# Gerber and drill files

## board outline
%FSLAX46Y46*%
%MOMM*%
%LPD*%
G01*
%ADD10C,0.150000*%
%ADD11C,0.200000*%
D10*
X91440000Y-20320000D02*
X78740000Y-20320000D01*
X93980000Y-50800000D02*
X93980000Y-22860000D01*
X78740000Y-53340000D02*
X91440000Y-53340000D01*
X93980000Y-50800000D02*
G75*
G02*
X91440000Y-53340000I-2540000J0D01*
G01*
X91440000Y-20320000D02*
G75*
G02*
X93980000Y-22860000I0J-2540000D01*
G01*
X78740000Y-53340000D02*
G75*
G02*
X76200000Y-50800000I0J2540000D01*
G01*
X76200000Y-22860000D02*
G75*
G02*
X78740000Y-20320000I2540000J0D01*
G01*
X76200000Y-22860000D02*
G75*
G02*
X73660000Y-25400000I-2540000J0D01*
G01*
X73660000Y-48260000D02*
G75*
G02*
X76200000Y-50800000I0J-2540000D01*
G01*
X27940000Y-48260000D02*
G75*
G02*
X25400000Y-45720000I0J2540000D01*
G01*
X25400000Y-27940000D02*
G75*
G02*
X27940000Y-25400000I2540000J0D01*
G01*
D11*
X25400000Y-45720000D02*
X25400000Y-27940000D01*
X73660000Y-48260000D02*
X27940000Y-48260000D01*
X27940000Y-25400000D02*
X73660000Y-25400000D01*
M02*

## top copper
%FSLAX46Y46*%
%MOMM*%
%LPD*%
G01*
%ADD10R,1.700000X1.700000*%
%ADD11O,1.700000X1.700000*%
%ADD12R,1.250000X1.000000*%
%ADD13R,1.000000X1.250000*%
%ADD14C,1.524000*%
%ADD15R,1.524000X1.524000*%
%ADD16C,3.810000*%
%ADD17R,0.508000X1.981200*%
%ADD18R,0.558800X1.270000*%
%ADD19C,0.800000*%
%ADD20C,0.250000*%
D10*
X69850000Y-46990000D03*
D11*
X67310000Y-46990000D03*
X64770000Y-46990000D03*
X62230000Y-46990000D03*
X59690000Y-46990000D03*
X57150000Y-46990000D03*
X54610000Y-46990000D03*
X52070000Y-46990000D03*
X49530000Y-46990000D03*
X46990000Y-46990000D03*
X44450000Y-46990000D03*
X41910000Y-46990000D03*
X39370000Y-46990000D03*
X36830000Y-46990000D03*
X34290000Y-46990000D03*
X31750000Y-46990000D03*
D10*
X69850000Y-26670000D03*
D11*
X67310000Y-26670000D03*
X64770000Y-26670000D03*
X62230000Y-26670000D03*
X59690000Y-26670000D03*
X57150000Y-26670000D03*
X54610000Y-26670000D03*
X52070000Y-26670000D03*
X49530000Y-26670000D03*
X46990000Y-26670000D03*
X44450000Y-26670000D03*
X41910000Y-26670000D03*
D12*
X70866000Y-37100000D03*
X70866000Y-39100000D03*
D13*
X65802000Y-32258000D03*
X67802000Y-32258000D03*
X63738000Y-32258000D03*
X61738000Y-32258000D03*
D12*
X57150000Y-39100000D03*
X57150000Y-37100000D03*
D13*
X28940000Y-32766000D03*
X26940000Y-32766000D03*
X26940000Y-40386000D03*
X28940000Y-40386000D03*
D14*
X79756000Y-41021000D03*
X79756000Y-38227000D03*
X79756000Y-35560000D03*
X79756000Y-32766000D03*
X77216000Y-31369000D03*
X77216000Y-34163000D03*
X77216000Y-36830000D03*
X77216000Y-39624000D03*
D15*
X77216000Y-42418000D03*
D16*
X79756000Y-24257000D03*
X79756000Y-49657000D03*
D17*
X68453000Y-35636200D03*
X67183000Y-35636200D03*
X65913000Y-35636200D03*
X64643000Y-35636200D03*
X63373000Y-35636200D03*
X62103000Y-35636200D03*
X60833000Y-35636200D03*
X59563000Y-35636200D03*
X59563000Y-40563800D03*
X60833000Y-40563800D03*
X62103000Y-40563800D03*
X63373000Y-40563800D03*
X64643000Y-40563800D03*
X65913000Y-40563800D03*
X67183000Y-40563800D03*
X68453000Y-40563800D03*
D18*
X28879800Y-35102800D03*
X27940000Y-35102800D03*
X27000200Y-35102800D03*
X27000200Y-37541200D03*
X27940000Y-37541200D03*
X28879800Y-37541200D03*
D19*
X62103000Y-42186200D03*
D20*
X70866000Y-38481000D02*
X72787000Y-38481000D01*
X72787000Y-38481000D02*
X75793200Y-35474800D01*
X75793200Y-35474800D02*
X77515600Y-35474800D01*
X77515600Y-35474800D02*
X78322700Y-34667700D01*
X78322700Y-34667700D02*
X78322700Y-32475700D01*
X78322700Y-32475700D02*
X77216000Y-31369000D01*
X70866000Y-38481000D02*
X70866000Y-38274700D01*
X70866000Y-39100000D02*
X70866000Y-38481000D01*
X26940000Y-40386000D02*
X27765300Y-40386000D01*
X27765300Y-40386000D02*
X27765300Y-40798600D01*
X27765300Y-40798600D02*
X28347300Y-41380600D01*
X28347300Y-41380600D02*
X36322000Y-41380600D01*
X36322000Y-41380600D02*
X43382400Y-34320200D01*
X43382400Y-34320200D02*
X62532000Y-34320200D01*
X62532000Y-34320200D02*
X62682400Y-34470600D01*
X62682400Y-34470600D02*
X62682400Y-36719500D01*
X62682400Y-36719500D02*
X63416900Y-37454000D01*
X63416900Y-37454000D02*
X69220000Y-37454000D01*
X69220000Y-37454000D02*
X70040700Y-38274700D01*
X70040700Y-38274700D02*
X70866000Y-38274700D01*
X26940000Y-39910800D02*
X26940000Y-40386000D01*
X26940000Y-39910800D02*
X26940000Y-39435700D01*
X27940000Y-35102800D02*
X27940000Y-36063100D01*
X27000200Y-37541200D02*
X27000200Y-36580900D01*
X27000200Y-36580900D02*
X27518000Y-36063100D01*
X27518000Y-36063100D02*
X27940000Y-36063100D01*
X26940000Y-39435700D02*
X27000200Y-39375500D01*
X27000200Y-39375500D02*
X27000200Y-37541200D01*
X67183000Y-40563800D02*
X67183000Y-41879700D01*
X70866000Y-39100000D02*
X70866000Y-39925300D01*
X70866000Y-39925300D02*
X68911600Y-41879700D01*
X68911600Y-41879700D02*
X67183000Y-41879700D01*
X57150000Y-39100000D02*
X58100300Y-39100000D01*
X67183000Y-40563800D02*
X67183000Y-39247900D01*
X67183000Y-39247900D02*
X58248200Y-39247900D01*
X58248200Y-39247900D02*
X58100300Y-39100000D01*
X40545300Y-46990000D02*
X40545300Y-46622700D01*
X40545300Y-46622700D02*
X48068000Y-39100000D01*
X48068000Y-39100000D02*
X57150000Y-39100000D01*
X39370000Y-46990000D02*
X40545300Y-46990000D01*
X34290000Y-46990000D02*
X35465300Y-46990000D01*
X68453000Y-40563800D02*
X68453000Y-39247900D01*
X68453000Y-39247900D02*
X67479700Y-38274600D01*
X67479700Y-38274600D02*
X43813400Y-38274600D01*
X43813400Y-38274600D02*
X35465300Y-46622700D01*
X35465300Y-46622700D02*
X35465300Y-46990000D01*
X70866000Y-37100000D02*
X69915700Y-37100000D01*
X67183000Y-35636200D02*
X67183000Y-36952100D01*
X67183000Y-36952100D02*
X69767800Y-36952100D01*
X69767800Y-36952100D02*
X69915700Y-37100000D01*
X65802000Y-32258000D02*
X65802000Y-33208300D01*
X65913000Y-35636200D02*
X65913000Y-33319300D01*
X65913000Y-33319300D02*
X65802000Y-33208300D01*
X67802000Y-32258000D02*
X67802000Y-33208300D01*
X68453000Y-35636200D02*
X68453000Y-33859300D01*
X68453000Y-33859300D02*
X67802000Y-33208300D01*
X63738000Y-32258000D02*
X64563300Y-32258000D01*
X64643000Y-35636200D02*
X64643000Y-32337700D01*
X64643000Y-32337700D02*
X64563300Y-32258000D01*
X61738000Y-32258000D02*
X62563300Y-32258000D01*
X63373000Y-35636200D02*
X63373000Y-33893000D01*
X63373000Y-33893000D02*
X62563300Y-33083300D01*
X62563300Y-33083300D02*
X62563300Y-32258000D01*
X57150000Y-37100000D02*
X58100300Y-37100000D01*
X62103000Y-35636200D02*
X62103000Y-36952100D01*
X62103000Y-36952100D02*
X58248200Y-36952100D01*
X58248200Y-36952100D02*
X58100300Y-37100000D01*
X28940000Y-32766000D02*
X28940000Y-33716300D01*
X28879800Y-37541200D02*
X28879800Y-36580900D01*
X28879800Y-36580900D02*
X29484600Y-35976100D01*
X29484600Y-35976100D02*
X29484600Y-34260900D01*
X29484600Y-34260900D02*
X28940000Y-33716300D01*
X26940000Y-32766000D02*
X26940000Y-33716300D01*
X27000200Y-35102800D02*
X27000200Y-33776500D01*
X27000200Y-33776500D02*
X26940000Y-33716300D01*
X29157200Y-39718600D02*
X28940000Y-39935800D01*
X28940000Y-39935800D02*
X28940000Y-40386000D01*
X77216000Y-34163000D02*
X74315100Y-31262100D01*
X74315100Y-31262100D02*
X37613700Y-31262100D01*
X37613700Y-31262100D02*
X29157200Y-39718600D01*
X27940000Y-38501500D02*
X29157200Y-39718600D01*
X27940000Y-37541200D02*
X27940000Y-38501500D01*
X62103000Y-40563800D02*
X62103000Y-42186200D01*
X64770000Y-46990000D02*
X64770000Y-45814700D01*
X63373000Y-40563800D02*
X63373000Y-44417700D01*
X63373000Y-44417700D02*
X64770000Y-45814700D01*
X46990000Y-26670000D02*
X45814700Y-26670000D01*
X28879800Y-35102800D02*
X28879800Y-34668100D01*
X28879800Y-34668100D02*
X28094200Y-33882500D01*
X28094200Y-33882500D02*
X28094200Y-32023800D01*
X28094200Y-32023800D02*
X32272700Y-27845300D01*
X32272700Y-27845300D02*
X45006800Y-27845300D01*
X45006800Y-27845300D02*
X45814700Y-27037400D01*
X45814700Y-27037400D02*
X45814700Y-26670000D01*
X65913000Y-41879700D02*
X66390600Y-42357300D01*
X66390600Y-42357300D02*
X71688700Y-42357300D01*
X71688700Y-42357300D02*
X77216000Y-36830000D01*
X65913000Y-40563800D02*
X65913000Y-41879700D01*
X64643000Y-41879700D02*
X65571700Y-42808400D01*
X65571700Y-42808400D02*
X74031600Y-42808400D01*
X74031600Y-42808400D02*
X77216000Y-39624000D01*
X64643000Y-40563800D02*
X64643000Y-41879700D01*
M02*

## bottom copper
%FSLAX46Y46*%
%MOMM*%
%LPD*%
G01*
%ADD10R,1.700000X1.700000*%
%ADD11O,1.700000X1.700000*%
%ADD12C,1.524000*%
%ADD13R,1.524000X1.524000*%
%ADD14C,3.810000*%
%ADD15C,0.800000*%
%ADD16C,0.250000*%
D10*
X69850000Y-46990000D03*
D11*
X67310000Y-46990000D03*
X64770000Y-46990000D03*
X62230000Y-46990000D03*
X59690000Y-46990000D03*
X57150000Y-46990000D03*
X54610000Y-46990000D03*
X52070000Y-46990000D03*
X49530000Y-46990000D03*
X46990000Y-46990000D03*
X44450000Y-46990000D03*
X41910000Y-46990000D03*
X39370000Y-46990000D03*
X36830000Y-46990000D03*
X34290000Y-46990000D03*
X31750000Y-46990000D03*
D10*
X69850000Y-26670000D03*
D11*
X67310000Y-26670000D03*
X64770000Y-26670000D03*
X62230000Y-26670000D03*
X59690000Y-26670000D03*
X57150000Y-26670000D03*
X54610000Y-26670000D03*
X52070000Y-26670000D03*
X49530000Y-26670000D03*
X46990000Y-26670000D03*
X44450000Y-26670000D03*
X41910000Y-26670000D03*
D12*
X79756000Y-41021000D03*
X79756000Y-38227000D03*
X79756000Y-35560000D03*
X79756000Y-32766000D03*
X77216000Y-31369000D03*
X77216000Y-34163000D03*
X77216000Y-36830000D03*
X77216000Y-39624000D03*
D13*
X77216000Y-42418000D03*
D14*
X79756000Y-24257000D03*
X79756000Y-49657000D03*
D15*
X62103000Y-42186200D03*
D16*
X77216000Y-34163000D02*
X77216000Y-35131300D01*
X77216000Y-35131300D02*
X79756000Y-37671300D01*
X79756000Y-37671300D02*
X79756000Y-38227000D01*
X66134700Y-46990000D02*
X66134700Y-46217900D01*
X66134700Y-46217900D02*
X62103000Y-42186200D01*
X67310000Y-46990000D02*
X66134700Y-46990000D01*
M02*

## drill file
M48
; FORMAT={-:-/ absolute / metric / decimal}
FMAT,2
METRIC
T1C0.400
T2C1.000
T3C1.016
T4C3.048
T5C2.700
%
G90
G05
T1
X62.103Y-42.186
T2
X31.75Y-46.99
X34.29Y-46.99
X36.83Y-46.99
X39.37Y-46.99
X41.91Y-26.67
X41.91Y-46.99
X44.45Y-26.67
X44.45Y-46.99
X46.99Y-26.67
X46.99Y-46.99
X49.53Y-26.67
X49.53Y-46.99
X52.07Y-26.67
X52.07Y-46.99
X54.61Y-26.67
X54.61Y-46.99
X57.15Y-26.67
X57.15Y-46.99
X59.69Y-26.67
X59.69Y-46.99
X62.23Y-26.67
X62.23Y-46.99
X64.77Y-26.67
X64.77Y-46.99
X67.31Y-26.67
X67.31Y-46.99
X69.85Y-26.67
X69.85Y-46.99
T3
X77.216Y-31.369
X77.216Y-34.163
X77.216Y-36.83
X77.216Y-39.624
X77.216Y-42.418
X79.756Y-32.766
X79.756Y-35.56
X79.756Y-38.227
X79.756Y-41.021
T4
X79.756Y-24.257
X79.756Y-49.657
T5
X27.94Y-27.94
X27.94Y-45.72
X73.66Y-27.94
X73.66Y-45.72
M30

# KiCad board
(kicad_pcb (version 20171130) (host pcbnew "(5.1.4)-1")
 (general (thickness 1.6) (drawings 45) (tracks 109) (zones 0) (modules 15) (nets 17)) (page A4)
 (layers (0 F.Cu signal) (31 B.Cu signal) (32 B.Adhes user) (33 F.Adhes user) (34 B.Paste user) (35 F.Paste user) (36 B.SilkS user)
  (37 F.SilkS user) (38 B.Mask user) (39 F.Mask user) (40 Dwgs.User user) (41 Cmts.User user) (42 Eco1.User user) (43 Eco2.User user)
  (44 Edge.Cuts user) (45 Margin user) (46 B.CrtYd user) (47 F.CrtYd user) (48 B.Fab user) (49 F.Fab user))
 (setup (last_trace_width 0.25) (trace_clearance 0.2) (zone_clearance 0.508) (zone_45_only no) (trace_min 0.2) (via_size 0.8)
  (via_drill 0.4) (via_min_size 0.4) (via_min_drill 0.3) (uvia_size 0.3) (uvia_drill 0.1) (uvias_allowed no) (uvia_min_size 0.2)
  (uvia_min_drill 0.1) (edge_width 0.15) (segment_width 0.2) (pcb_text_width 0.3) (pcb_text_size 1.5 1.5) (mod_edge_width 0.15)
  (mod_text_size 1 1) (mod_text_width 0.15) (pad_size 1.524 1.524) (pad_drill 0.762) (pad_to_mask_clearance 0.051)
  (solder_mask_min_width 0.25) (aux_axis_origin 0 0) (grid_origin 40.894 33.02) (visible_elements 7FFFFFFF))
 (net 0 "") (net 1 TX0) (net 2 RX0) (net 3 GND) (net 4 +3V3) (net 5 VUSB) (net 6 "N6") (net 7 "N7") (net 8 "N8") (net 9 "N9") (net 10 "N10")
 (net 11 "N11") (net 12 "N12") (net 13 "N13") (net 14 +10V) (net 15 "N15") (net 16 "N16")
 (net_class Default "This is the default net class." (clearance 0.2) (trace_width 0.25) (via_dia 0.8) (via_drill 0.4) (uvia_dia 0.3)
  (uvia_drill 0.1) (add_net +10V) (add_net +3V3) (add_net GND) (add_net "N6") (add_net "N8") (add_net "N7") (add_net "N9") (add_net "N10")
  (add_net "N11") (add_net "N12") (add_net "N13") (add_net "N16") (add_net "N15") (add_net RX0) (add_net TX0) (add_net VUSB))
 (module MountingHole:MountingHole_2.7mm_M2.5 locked (layer F.Cu) (at 73.66 27.94)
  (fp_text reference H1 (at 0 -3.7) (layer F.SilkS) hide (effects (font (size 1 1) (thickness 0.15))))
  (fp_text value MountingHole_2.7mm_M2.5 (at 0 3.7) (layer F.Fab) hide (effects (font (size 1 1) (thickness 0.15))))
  (pad 1 np_thru_hole circle (at 0 0) (size 2.7 2.7) (drill 2.7) (layers *.Cu *.Mask)))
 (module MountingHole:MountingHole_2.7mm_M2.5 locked (layer F.Cu) (at 73.66 45.72)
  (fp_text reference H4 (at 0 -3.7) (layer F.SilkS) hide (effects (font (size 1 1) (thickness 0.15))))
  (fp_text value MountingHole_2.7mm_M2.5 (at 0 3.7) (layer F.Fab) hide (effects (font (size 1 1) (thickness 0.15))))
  (pad 1 np_thru_hole circle (at 0 0) (size 2.7 2.7) (drill 2.7) (layers *.Cu *.Mask)))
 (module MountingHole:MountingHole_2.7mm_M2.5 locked (layer F.Cu) (at 27.94 45.72)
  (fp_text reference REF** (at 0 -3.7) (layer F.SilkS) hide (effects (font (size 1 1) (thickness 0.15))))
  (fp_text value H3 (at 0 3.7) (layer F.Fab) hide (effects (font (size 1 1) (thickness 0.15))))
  (pad 1 np_thru_hole circle (at 0 0) (size 2.7 2.7) (drill 2.7) (layers *.Cu *.Mask)))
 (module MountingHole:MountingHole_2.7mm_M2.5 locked (layer F.Cu) (at 27.94 27.94)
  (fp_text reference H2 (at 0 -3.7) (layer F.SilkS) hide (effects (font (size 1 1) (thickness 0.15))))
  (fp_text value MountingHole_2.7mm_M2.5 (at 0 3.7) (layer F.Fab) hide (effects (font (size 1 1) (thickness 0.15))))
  (pad 1 np_thru_hole circle (at 0 0) (size 2.7 2.7) (drill 2.7) (layers *.Cu *.Mask)))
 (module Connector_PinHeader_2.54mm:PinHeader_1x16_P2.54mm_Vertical (layer B.Cu) (at 69.85 46.99 90)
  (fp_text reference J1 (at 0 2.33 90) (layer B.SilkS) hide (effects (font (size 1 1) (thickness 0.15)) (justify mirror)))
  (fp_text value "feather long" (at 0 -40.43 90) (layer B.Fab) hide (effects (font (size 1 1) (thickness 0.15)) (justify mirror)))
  (pad 1 thru_hole rect (at 0 0 90) (size 1.7 1.7) (drill 1) (layers *.Cu *.Mask))
  (pad 2 thru_hole oval (at 0 -2.54 90) (size 1.7 1.7) (drill 1) (layers *.Cu *.Mask) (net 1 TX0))
  (pad 3 thru_hole oval (at 0 -5.08 90) (size 1.7 1.7) (drill 1) (layers *.Cu *.Mask) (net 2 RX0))
  (pad 4 thru_hole oval (at 0 -7.62 90) (size 1.7 1.7) (drill 1) (layers *.Cu *.Mask))
  (pad 5 thru_hole oval (at 0 -10.16 90) (size 1.7 1.7) (drill 1) (layers *.Cu *.Mask))
  (pad 6 thru_hole oval (at 0 -12.7 90) (size 1.7 1.7) (drill 1) (layers *.Cu *.Mask))
  (pad 7 thru_hole oval (at 0 -15.24 90) (size 1.7 1.7) (drill 1) (layers *.Cu *.Mask))
  (pad 8 thru_hole oval (at 0 -17.78 90) (size 1.7 1.7) (drill 1) (layers *.Cu *.Mask))
  (pad 9 thru_hole oval (at 0 -20.32 90) (size 1.7 1.7) (drill 1) (layers *.Cu *.Mask))
  (pad 10 thru_hole oval (at 0 -22.86 90) (size 1.7 1.7) (drill 1) (layers *.Cu *.Mask))
  (pad 11 thru_hole oval (at 0 -25.4 90) (size 1.7 1.7) (drill 1) (layers *.Cu *.Mask))
  (pad 12 thru_hole oval (at 0 -27.94 90) (size 1.7 1.7) (drill 1) (layers *.Cu *.Mask))
  (pad 13 thru_hole oval (at 0 -30.48 90) (size 1.7 1.7) (drill 1) (layers *.Cu *.Mask) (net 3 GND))
  (pad 14 thru_hole oval (at 0 -33.02 90) (size 1.7 1.7) (drill 1) (layers *.Cu *.Mask))
  (pad 15 thru_hole oval (at 0 -35.56 90) (size 1.7 1.7) (drill 1) (layers *.Cu *.Mask) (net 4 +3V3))
  (pad 16 thru_hole oval (at 0 -38.1 90) (size 1.7 1.7) (drill 1) (layers *.Cu *.Mask)))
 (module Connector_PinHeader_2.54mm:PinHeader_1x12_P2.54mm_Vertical (layer B.Cu) (at 69.85 26.67 90)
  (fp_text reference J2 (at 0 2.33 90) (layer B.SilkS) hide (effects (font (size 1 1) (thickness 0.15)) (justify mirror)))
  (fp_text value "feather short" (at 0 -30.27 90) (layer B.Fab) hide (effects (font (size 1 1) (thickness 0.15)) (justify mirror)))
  (pad 1 thru_hole rect (at 0 0 90) (size 1.7 1.7) (drill 1) (layers *.Cu *.Mask))
  (pad 2 thru_hole oval (at 0 -2.54 90) (size 1.7 1.7) (drill 1) (layers *.Cu *.Mask))
  (pad 3 thru_hole oval (at 0 -5.08 90) (size 1.7 1.7) (drill 1) (layers *.Cu *.Mask))
  (pad 4 thru_hole oval (at 0 -7.62 90) (size 1.7 1.7) (drill 1) (layers *.Cu *.Mask))
  (pad 5 thru_hole oval (at 0 -10.16 90) (size 1.7 1.7) (drill 1) (layers *.Cu *.Mask))
  (pad 6 thru_hole oval (at 0 -12.7 90) (size 1.7 1.7) (drill 1) (layers *.Cu *.Mask))
  (pad 7 thru_hole oval (at 0 -15.24 90) (size 1.7 1.7) (drill 1) (layers *.Cu *.Mask))
  (pad 8 thru_hole oval (at 0 -17.78 90) (size 1.7 1.7) (drill 1) (layers *.Cu *.Mask))
  (pad 9 thru_hole oval (at 0 -20.32 90) (size 1.7 1.7) (drill 1) (layers *.Cu *.Mask))
  (pad 10 thru_hole oval (at 0 -22.86 90) (size 1.7 1.7) (drill 1) (layers *.Cu *.Mask) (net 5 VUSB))
  (pad 11 thru_hole oval (at 0 -25.4 90) (size 1.7 1.7) (drill 1) (layers *.Cu *.Mask))
  (pad 12 thru_hole oval (at 0 -27.94 90) (size 1.7 1.7) (drill 1) (layers *.Cu *.Mask)))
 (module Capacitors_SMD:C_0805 (layer F.Cu) (at 70.866 38.1 270)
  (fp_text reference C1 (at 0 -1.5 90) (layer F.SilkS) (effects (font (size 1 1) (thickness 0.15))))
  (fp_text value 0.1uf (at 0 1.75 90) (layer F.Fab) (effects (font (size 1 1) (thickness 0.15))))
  (pad 1 smd rect (at -1 0 270) (size 1 1.25) (layers F.Cu F.Paste F.Mask) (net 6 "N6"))
  (pad 2 smd rect (at 1 0 270) (size 1 1.25) (layers F.Cu F.Paste F.Mask) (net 3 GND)))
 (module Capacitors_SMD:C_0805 (layer F.Cu) (at 66.802 32.258 180)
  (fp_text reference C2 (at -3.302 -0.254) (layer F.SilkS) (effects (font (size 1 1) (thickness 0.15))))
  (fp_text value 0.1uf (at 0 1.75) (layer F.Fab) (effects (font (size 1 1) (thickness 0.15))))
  (pad 2 smd rect (at 1 0 180) (size 1 1.25) (layers F.Cu F.Paste F.Mask) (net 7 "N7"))
  (pad 1 smd rect (at -1 0 180) (size 1 1.25) (layers F.Cu F.Paste F.Mask) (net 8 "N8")))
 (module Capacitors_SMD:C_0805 (layer F.Cu) (at 62.738 32.258 180)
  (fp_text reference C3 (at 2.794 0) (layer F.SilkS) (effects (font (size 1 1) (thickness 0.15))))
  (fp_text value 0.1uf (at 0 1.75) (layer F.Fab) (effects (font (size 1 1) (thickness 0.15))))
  (pad 1 smd rect (at -1 0 180) (size 1 1.25) (layers F.Cu F.Paste F.Mask) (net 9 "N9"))
  (pad 2 smd rect (at 1 0 180) (size 1 1.25) (layers F.Cu F.Paste F.Mask) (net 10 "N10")))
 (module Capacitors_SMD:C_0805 (layer F.Cu) (at 57.15 38.1 270)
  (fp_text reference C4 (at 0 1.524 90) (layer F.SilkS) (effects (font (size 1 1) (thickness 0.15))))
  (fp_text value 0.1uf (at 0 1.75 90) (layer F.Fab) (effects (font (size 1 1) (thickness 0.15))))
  (pad 2 smd rect (at 1 0 270) (size 1 1.25) (layers F.Cu F.Paste F.Mask) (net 3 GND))
  (pad 1 smd rect (at -1 0 270) (size 1 1.25) (layers F.Cu F.Paste F.Mask) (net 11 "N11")))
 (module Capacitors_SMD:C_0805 (layer F.Cu) (at 27.94 32.766 180)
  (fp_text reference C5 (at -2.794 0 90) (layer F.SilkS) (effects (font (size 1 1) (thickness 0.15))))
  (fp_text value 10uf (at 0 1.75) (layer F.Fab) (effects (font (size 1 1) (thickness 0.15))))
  (pad 1 smd rect (at -1 0 180) (size 1 1.25) (layers F.Cu F.Paste F.Mask) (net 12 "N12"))
  (pad 2 smd rect (at 1 0 180) (size 1 1.25) (layers F.Cu F.Paste F.Mask) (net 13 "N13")))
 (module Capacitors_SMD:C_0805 (layer F.Cu) (at 27.94 40.386 180)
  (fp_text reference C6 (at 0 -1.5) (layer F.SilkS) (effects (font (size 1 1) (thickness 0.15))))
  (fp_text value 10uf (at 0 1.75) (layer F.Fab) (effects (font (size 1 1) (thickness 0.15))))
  (pad 2 smd rect (at 1 0 180) (size 1 1.25) (layers F.Cu F.Paste F.Mask) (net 3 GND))
  (pad 1 smd rect (at -1 0 180) (size 1 1.25) (layers F.Cu F.Paste F.Mask) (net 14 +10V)))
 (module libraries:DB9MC (layer F.Cu) (at 78.486 36.83 270)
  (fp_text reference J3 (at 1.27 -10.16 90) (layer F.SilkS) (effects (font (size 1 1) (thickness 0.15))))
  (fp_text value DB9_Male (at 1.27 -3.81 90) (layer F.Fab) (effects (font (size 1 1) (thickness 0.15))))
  (pad 6 thru_hole circle (at 4.191 -1.27 270) (size 1.524 1.524) (drill 1.016) (layers *.Cu *.Mask F.SilkS))
  (pad 7 thru_hole circle (at 1.397 -1.27 270) (size 1.524 1.524) (drill 1.016) (layers *.Cu *.Mask F.SilkS) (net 14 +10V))
  (pad 8 thru_hole circle (at -1.27 -1.27 270) (size 1.524 1.524) (drill 1.016) (layers *.Cu *.Mask F.SilkS))
  (pad 9 thru_hole circle (at -4.064 -1.27 270) (size 1.524 1.524) (drill 1.016) (layers *.Cu *.Mask F.SilkS))
  (pad 5 thru_hole circle (at -5.461 1.27 270) (size 1.524 1.524) (drill 1.016) (layers *.Cu *.Mask F.SilkS) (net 3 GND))
  (pad 4 thru_hole circle (at -2.667 1.27 270) (size 1.524 1.524) (drill 1.016) (layers *.Cu *.Mask F.SilkS) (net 14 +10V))
  (pad 3 thru_hole circle (at 0 1.27 270) (size 1.524 1.524) (drill 1.016) (layers *.Cu *.Mask F.SilkS) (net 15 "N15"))
  (pad 2 thru_hole circle (at 2.794 1.27 270) (size 1.524 1.524) (drill 1.016) (layers *.Cu *.Mask F.SilkS) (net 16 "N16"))
  (pad 1 thru_hole rect (at 5.588 1.27 270) (size 1.524 1.524) (drill 1.016) (layers *.Cu *.Mask F.SilkS))
  (pad "" thru_hole circle (at -12.573 -1.27 270) (size 3.81 3.81) (drill 3.048) (layers *.Cu *.Mask F.SilkS))
  (pad "" thru_hole circle (at 12.827 -1.27 270) (size 3.81 3.81) (drill 3.048) (layers *.Cu *.Mask F.SilkS)))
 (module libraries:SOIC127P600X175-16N (layer F.Cu) (at 64.008 38.1 270)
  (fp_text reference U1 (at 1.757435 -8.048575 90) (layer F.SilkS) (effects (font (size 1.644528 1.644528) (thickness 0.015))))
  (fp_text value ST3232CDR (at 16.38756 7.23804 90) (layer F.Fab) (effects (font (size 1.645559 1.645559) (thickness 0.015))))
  (pad 1 smd rect (at -2.4638 -4.445 270) (size 1.9812 0.508) (layers F.Cu F.Paste F.Mask) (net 8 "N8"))
  (pad 2 smd rect (at -2.4638 -3.175 270) (size 1.9812 0.508) (layers F.Cu F.Paste F.Mask) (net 6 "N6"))
  (pad 3 smd rect (at -2.4638 -1.905 270) (size 1.9812 0.508) (layers F.Cu F.Paste F.Mask) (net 7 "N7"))
  (pad 4 smd rect (at -2.4638 -0.635 270) (size 1.9812 0.508) (layers F.Cu F.Paste F.Mask) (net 9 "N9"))
  (pad 5 smd rect (at -2.4638 0.635 270) (size 1.9812 0.508) (layers F.Cu F.Paste F.Mask) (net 10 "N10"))
  (pad 6 smd rect (at -2.4638 1.905 270) (size 1.9812 0.508) (layers F.Cu F.Paste F.Mask) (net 11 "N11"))
  (pad 7 smd rect (at -2.4638 3.175 270) (size 1.9812 0.508) (layers F.Cu F.Paste F.Mask))
  (pad 8 smd rect (at -2.4638 4.445 270) (size 1.9812 0.508) (layers F.Cu F.Paste F.Mask))
  (pad 9 smd rect (at 2.4638 4.445 270) (size 1.9812 0.508) (layers F.Cu F.Paste F.Mask))
  (pad 10 smd rect (at 2.4638 3.175 270) (size 1.9812 0.508) (layers F.Cu F.Paste F.Mask))
  (pad 11 smd rect (at 2.4638 1.905 270) (size 1.9812 0.508) (layers F.Cu F.Paste F.Mask) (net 1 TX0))
  (pad 12 smd rect (at 2.4638 0.635 270) (size 1.9812 0.508) (layers F.Cu F.Paste F.Mask) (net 2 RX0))
  (pad 13 smd rect (at 2.4638 -0.635 270) (size 1.9812 0.508) (layers F.Cu F.Paste F.Mask) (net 16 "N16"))
  (pad 14 smd rect (at 2.4638 -1.905 270) (size 1.9812 0.508) (layers F.Cu F.Paste F.Mask) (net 15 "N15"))
  (pad 15 smd rect (at 2.4638 -3.175 270) (size 1.9812 0.508) (layers F.Cu F.Paste F.Mask) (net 3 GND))
  (pad 16 smd rect (at 2.4638 -4.445 270) (size 1.9812 0.508) (layers F.Cu F.Paste F.Mask) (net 4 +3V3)))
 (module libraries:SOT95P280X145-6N (layer F.Cu) (at 27.94 36.322 270)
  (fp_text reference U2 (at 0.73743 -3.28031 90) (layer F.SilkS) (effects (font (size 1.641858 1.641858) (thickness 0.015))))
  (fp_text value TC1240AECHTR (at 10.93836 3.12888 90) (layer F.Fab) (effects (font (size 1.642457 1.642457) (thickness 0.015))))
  (pad 1 smd rect (at -1.2192 -0.9398 270) (size 1.27 0.5588) (layers F.Cu F.Paste F.Mask) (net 5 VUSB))
  (pad 2 smd rect (at -1.2192 0 270) (size 1.27 0.5588) (layers F.Cu F.Paste F.Mask) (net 3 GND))
  (pad 3 smd rect (at -1.2192 0.9398 270) (size 1.27 0.5588) (layers F.Cu F.Paste F.Mask) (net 13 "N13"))
  (pad 4 smd rect (at 1.2192 0.9398 270) (size 1.27 0.5588) (layers F.Cu F.Paste F.Mask) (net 3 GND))
  (pad 5 smd rect (at 1.2192 0 270) (size 1.27 0.5588) (layers F.Cu F.Paste F.Mask) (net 14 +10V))
  (pad 6 smd rect (at 1.2192 -0.9398 270) (size 1.27 0.5588) (layers F.Cu F.Paste F.Mask) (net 12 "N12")))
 (gr_line (start 91.44 20.32) (end 78.74 20.32) (layer Edge.Cuts) (width 0.15))
 (gr_line (start 93.98 50.8) (end 93.98 22.86) (layer Edge.Cuts) (width 0.15))
 (gr_line (start 78.74 53.34) (end 91.44 53.34) (layer Edge.Cuts) (width 0.15))
 (gr_arc (start 91.44 50.8) (end 91.44 53.34) (angle -90) (layer Edge.Cuts) (width 0.15))
 (gr_arc (start 91.44 22.86) (end 93.98 22.86) (angle -90) (layer Edge.Cuts) (width 0.15))
 (gr_arc (start 78.74 50.8) (end 76.2 50.8) (angle -90) (layer Edge.Cuts) (width 0.15))
 (gr_arc (start 78.74 22.86) (end 78.74 20.32) (angle -90) (layer Edge.Cuts) (width 0.15))
 (gr_arc (start 73.66 22.86) (end 73.66 25.4) (angle -90) (layer Edge.Cuts) (width 0.15))
 (gr_arc (start 73.66 50.8) (end 76.2 50.8) (angle -90) (layer Edge.Cuts) (width 0.15))
 (gr_arc (start 27.94 45.72) (end 25.4 45.72) (angle -90) (layer Edge.Cuts) (width 0.15))
 (gr_arc (start 27.94 27.94) (end 27.94 25.4) (angle -90) (layer Edge.Cuts) (width 0.15))
 (gr_line (start 25.4 45.72) (end 25.4 27.94) (layer Edge.Cuts) (width 0.2))
 (gr_line (start 73.66 48.26) (end 27.94 48.26) (layer Edge.Cuts) (width 0.2))
 (gr_line (start 27.94 25.4) (end 73.66 25.4) (layer Edge.Cuts) (width 0.2))
 (segment (start 70.866 38.481) (end 72.787 38.481) (width 0.25) (layer F.Cu) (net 3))
 (segment (start 72.787 38.481) (end 75.7932 35.4748) (width 0.25) (layer F.Cu) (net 3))
 (segment (start 75.7932 35.4748) (end 77.5156 35.4748) (width 0.25) (layer F.Cu) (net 3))
 (segment (start 77.5156 35.4748) (end 78.3227 34.6677) (width 0.25) (layer F.Cu) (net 3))
 (segment (start 78.3227 34.6677) (end 78.3227 32.4757) (width 0.25) (layer F.Cu) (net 3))
 (segment (start 78.3227 32.4757) (end 77.216 31.369) (width 0.25) (layer F.Cu) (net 3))
 (segment (start 70.866 38.481) (end 70.866 38.2747) (width 0.25) (layer F.Cu) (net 3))
 (segment (start 70.866 39.1) (end 70.866 38.481) (width 0.25) (layer F.Cu) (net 3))
 (segment (start 26.94 40.386) (end 27.7653 40.386) (width 0.25) (layer F.Cu) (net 3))
 (segment (start 27.7653 40.386) (end 27.7653 40.7986) (width 0.25) (layer F.Cu) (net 3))
 (segment (start 27.7653 40.7986) (end 28.3473 41.3806) (width 0.25) (layer F.Cu) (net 3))
 (segment (start 28.3473 41.3806) (end 36.322 41.3806) (width 0.25) (layer F.Cu) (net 3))
 (segment (start 36.322 41.3806) (end 43.3824 34.3202) (width 0.25) (layer F.Cu) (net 3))
 (segment (start 43.3824 34.3202) (end 62.532 34.3202) (width 0.25) (layer F.Cu) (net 3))
 (segment (start 62.532 34.3202) (end 62.6824 34.4706) (width 0.25) (layer F.Cu) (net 3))
 (segment (start 62.6824 34.4706) (end 62.6824 36.7195) (width 0.25) (layer F.Cu) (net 3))
 (segment (start 62.6824 36.7195) (end 63.4169 37.454) (width 0.25) (layer F.Cu) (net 3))
 (segment (start 63.4169 37.454) (end 69.22 37.454) (width 0.25) (layer F.Cu) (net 3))
 (segment (start 69.22 37.454) (end 70.0407 38.2747) (width 0.25) (layer F.Cu) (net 3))
 (segment (start 70.0407 38.2747) (end 70.866 38.2747) (width 0.25) (layer F.Cu) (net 3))
 (segment (start 26.94 39.9108) (end 26.94 40.386) (width 0.25) (layer F.Cu) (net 3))
 (segment (start 26.94 39.9108) (end 26.94 39.4357) (width 0.25) (layer F.Cu) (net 3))
 (segment (start 27.94 35.1028) (end 27.94 36.0631) (width 0.25) (layer F.Cu) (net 3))
 (segment (start 27.0002 37.5412) (end 27.0002 36.5809) (width 0.25) (layer F.Cu) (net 3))
 (segment (start 27.0002 36.5809) (end 27.518 36.0631) (width 0.25) (layer F.Cu) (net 3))
 (segment (start 27.518 36.0631) (end 27.94 36.0631) (width 0.25) (layer F.Cu) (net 3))
 (segment (start 26.94 39.4357) (end 27.0002 39.3755) (width 0.25) (layer F.Cu) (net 3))
 (segment (start 27.0002 39.3755) (end 27.0002 37.5412) (width 0.25) (layer F.Cu) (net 3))
 (segment (start 67.183 40.5638) (end 67.183 41.8797) (width 0.25) (layer F.Cu) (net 3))
 (segment (start 70.866 39.1) (end 70.866 39.9253) (width 0.25) (layer F.Cu) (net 3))
 (segment (start 70.866 39.9253) (end 68.9116 41.8797) (width 0.25) (layer F.Cu) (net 3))
 (segment (start 68.9116 41.8797) (end 67.183 41.8797) (width 0.25) (layer F.Cu) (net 3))
 (segment (start 57.15 39.1) (end 58.1003 39.1) (width 0.25) (layer F.Cu) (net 3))
 (segment (start 67.183 40.5638) (end 67.183 39.2479) (width 0.25) (layer F.Cu) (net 3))
 (segment (start 67.183 39.2479) (end 58.2482 39.2479) (width 0.25) (layer F.Cu) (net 3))
 (segment (start 58.2482 39.2479) (end 58.1003 39.1) (width 0.25) (layer F.Cu) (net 3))
 (segment (start 40.5453 46.99) (end 40.5453 46.6227) (width 0.25) (layer F.Cu) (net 3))
 (segment (start 40.5453 46.6227) (end 48.068 39.1) (width 0.25) (layer F.Cu) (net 3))
 (segment (start 48.068 39.1) (end 57.15 39.1) (width 0.25) (layer F.Cu) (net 3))
 (segment (start 39.37 46.99) (end 40.5453 46.99) (width 0.25) (layer F.Cu) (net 3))
 (segment (start 34.29 46.99) (end 35.4653 46.99) (width 0.25) (layer F.Cu) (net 4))
 (segment (start 68.453 40.5638) (end 68.453 39.2479) (width 0.25) (layer F.Cu) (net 4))
 (segment (start 68.453 39.2479) (end 67.4797 38.2746) (width 0.25) (layer F.Cu) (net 4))
 (segment (start 67.4797 38.2746) (end 43.8134 38.2746) (width 0.25) (layer F.Cu) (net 4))
 (segment (start 43.8134 38.2746) (end 35.4653 46.6227) (width 0.25) (layer F.Cu) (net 4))
 (segment (start 35.4653 46.6227) (end 35.4653 46.99) (width 0.25) (layer F.Cu) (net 4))
 (segment (start 70.866 37.1) (end 69.9157 37.1) (width 0.25) (layer F.Cu) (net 6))
 (segment (start 67.183 35.6362) (end 67.183 36.9521) (width 0.25) (layer F.Cu) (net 6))
 (segment (start 67.183 36.9521) (end 69.7678 36.9521) (width 0.25) (layer F.Cu) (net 6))
 (segment (start 69.7678 36.9521) (end 69.9157 37.1) (width 0.25) (layer F.Cu) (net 6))
 (segment (start 65.802 32.258) (end 65.802 33.2083) (width 0.25) (layer F.Cu) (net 7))
 (segment (start 65.913 35.6362) (end 65.913 33.3193) (width 0.25) (layer F.Cu) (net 7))
 (segment (start 65.913 33.3193) (end 65.802 33.2083) (width 0.25) (layer F.Cu) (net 7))
 (segment (start 67.802 32.258) (end 67.802 33.2083) (width 0.25) (layer F.Cu) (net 8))
 (segment (start 68.453 35.6362) (end 68.453 33.8593) (width 0.25) (layer F.Cu) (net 8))
 (segment (start 68.453 33.8593) (end 67.802 33.2083) (width 0.25) (layer F.Cu) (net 8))
 (segment (start 63.738 32.258) (end 64.5633 32.258) (width 0.25) (layer F.Cu) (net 9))
 (segment (start 64.643 35.6362) (end 64.643 32.3377) (width 0.25) (layer F.Cu) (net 9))
 (segment (start 64.643 32.3377) (end 64.5633 32.258) (width 0.25) (layer F.Cu) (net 9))
 (segment (start 61.738 32.258) (end 62.5633 32.258) (width 0.25) (layer F.Cu) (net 10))
 (segment (start 63.373 35.6362) (end 63.373 33.893) (width 0.25) (layer F.Cu) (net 10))
 (segment (start 63.373 33.893) (end 62.5633 33.0833) (width 0.25) (layer F.Cu) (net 10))
 (segment (start 62.5633 33.0833) (end 62.5633 32.258) (width 0.25) (layer F.Cu) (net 10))
 (segment (start 57.15 37.1) (end 58.1003 37.1) (width 0.25) (layer F.Cu) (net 11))
 (segment (start 62.103 35.6362) (end 62.103 36.9521) (width 0.25) (layer F.Cu) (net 11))
 (segment (start 62.103 36.9521) (end 58.2482 36.9521) (width 0.25) (layer F.Cu) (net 11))
 (segment (start 58.2482 36.9521) (end 58.1003 37.1) (width 0.25) (layer F.Cu) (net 11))
 (segment (start 28.94 32.766) (end 28.94 33.7163) (width 0.25) (layer F.Cu) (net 12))
 (segment (start 28.8798 37.5412) (end 28.8798 36.5809) (width 0.25) (layer F.Cu) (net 12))
 (segment (start 28.8798 36.5809) (end 29.4846 35.9761) (width 0.25) (layer F.Cu) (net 12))
 (segment (start 29.4846 35.9761) (end 29.4846 34.2609) (width 0.25) (layer F.Cu) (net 12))
 (segment (start 29.4846 34.2609) (end 28.94 33.7163) (width 0.25) (layer F.Cu) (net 12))
 (segment (start 26.94 32.766) (end 26.94 33.7163) (width 0.25) (layer F.Cu) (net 13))
 (segment (start 27.0002 35.1028) (end 27.0002 33.7765) (width 0.25) (layer F.Cu) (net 13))
 (segment (start 27.0002 33.7765) (end 26.94 33.7163) (width 0.25) (layer F.Cu) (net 13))
 (segment (start 29.1572 39.7186) (end 28.94 39.9358) (width 0.25) (layer F.Cu) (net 14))
 (segment (start 28.94 39.9358) (end 28.94 40.386) (width 0.25) (layer F.Cu) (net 14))
 (segment (start 77.216 34.163) (end 74.3151 31.2621) (width 0.25) (layer F.Cu) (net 14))
 (segment (start 74.3151 31.2621) (end 37.6137 31.2621) (width 0.25) (layer F.Cu) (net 14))
 (segment (start 37.6137 31.2621) (end 29.1572 39.7186) (width 0.25) (layer F.Cu) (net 14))
 (segment (start 27.94 38.5015) (end 29.1572 39.7186) (width 0.25) (layer F.Cu) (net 14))
 (segment (start 27.94 37.5412) (end 27.94 38.5015) (width 0.25) (layer F.Cu) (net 14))
 (segment (start 77.216 34.163) (end 77.216 35.1313) (width 0.25) (layer B.Cu) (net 14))
 (segment (start 77.216 35.1313) (end 79.756 37.6713) (width 0.25) (layer B.Cu) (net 14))
 (segment (start 79.756 37.6713) (end 79.756 38.227) (width 0.25) (layer B.Cu) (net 14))
 (segment (start 62.103 40.5638) (end 62.103 42.1862) (width 0.25) (layer F.Cu) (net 1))
 (segment (start 66.1347 46.99) (end 66.1347 46.2179) (width 0.25) (layer B.Cu) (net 1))
 (segment (start 66.1347 46.2179) (end 62.103 42.1862) (width 0.25) (layer B.Cu) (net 1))
 (segment (start 67.31 46.99) (end 66.1347 46.99) (width 0.25) (layer B.Cu) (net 1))
 (via (at 62.103 42.1862) (size 0.8) (layers F.Cu B.Cu) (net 1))
 (segment (start 64.77 46.99) (end 64.77 45.8147) (width 0.25) (layer F.Cu) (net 2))
 (segment (start 63.373 40.5638) (end 63.373 44.4177) (width 0.25) (layer F.Cu) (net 2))
 (segment (start 63.373 44.4177) (end 64.77 45.8147) (width 0.25) (layer F.Cu) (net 2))
 (segment (start 46.99 26.67) (end 45.8147 26.67) (width 0.25) (layer F.Cu) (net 5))
 (segment (start 28.8798 35.1028) (end 28.8798 34.6681) (width 0.25) (layer F.Cu) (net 5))
 (segment (start 28.8798 34.6681) (end 28.0942 33.8825) (width 0.25) (layer F.Cu) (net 5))
 (segment (start 28.0942 33.8825) (end 28.0942 32.0238) (width 0.25) (layer F.Cu) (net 5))
 (segment (start 28.0942 32.0238) (end 32.2727 27.8453) (width 0.25) (layer F.Cu) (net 5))
 (segment (start 32.2727 27.8453) (end 45.0068 27.8453) (width 0.25) (layer F.Cu) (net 5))
 (segment (start 45.0068 27.8453) (end 45.8147 27.0374) (width 0.25) (layer F.Cu) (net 5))
 (segment (start 45.8147 27.0374) (end 45.8147 26.67) (width 0.25) (layer F.Cu) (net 5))
 (segment (start 65.913 41.8797) (end 66.3906 42.3573) (width 0.25) (layer F.Cu) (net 15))
 (segment (start 66.3906 42.3573) (end 71.6887 42.3573) (width 0.25) (layer F.Cu) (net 15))
 (segment (start 71.6887 42.3573) (end 77.216 36.83) (width 0.25) (layer F.Cu) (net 15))
 (segment (start 65.913 40.5638) (end 65.913 41.8797) (width 0.25) (layer F.Cu) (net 15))
 (segment (start 64.643 41.8797) (end 65.5717 42.8084) (width 0.25) (layer F.Cu) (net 16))
 (segment (start 65.5717 42.8084) (end 74.0316 42.8084) (width 0.25) (layer F.Cu) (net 16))
 (segment (start 74.0316 42.8084) (end 77.216 39.624) (width 0.25) (layer F.Cu) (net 16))
 (segment (start 64.643 40.5638) (end 64.643 41.8797) (width 0.25) (layer F.Cu) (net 16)))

